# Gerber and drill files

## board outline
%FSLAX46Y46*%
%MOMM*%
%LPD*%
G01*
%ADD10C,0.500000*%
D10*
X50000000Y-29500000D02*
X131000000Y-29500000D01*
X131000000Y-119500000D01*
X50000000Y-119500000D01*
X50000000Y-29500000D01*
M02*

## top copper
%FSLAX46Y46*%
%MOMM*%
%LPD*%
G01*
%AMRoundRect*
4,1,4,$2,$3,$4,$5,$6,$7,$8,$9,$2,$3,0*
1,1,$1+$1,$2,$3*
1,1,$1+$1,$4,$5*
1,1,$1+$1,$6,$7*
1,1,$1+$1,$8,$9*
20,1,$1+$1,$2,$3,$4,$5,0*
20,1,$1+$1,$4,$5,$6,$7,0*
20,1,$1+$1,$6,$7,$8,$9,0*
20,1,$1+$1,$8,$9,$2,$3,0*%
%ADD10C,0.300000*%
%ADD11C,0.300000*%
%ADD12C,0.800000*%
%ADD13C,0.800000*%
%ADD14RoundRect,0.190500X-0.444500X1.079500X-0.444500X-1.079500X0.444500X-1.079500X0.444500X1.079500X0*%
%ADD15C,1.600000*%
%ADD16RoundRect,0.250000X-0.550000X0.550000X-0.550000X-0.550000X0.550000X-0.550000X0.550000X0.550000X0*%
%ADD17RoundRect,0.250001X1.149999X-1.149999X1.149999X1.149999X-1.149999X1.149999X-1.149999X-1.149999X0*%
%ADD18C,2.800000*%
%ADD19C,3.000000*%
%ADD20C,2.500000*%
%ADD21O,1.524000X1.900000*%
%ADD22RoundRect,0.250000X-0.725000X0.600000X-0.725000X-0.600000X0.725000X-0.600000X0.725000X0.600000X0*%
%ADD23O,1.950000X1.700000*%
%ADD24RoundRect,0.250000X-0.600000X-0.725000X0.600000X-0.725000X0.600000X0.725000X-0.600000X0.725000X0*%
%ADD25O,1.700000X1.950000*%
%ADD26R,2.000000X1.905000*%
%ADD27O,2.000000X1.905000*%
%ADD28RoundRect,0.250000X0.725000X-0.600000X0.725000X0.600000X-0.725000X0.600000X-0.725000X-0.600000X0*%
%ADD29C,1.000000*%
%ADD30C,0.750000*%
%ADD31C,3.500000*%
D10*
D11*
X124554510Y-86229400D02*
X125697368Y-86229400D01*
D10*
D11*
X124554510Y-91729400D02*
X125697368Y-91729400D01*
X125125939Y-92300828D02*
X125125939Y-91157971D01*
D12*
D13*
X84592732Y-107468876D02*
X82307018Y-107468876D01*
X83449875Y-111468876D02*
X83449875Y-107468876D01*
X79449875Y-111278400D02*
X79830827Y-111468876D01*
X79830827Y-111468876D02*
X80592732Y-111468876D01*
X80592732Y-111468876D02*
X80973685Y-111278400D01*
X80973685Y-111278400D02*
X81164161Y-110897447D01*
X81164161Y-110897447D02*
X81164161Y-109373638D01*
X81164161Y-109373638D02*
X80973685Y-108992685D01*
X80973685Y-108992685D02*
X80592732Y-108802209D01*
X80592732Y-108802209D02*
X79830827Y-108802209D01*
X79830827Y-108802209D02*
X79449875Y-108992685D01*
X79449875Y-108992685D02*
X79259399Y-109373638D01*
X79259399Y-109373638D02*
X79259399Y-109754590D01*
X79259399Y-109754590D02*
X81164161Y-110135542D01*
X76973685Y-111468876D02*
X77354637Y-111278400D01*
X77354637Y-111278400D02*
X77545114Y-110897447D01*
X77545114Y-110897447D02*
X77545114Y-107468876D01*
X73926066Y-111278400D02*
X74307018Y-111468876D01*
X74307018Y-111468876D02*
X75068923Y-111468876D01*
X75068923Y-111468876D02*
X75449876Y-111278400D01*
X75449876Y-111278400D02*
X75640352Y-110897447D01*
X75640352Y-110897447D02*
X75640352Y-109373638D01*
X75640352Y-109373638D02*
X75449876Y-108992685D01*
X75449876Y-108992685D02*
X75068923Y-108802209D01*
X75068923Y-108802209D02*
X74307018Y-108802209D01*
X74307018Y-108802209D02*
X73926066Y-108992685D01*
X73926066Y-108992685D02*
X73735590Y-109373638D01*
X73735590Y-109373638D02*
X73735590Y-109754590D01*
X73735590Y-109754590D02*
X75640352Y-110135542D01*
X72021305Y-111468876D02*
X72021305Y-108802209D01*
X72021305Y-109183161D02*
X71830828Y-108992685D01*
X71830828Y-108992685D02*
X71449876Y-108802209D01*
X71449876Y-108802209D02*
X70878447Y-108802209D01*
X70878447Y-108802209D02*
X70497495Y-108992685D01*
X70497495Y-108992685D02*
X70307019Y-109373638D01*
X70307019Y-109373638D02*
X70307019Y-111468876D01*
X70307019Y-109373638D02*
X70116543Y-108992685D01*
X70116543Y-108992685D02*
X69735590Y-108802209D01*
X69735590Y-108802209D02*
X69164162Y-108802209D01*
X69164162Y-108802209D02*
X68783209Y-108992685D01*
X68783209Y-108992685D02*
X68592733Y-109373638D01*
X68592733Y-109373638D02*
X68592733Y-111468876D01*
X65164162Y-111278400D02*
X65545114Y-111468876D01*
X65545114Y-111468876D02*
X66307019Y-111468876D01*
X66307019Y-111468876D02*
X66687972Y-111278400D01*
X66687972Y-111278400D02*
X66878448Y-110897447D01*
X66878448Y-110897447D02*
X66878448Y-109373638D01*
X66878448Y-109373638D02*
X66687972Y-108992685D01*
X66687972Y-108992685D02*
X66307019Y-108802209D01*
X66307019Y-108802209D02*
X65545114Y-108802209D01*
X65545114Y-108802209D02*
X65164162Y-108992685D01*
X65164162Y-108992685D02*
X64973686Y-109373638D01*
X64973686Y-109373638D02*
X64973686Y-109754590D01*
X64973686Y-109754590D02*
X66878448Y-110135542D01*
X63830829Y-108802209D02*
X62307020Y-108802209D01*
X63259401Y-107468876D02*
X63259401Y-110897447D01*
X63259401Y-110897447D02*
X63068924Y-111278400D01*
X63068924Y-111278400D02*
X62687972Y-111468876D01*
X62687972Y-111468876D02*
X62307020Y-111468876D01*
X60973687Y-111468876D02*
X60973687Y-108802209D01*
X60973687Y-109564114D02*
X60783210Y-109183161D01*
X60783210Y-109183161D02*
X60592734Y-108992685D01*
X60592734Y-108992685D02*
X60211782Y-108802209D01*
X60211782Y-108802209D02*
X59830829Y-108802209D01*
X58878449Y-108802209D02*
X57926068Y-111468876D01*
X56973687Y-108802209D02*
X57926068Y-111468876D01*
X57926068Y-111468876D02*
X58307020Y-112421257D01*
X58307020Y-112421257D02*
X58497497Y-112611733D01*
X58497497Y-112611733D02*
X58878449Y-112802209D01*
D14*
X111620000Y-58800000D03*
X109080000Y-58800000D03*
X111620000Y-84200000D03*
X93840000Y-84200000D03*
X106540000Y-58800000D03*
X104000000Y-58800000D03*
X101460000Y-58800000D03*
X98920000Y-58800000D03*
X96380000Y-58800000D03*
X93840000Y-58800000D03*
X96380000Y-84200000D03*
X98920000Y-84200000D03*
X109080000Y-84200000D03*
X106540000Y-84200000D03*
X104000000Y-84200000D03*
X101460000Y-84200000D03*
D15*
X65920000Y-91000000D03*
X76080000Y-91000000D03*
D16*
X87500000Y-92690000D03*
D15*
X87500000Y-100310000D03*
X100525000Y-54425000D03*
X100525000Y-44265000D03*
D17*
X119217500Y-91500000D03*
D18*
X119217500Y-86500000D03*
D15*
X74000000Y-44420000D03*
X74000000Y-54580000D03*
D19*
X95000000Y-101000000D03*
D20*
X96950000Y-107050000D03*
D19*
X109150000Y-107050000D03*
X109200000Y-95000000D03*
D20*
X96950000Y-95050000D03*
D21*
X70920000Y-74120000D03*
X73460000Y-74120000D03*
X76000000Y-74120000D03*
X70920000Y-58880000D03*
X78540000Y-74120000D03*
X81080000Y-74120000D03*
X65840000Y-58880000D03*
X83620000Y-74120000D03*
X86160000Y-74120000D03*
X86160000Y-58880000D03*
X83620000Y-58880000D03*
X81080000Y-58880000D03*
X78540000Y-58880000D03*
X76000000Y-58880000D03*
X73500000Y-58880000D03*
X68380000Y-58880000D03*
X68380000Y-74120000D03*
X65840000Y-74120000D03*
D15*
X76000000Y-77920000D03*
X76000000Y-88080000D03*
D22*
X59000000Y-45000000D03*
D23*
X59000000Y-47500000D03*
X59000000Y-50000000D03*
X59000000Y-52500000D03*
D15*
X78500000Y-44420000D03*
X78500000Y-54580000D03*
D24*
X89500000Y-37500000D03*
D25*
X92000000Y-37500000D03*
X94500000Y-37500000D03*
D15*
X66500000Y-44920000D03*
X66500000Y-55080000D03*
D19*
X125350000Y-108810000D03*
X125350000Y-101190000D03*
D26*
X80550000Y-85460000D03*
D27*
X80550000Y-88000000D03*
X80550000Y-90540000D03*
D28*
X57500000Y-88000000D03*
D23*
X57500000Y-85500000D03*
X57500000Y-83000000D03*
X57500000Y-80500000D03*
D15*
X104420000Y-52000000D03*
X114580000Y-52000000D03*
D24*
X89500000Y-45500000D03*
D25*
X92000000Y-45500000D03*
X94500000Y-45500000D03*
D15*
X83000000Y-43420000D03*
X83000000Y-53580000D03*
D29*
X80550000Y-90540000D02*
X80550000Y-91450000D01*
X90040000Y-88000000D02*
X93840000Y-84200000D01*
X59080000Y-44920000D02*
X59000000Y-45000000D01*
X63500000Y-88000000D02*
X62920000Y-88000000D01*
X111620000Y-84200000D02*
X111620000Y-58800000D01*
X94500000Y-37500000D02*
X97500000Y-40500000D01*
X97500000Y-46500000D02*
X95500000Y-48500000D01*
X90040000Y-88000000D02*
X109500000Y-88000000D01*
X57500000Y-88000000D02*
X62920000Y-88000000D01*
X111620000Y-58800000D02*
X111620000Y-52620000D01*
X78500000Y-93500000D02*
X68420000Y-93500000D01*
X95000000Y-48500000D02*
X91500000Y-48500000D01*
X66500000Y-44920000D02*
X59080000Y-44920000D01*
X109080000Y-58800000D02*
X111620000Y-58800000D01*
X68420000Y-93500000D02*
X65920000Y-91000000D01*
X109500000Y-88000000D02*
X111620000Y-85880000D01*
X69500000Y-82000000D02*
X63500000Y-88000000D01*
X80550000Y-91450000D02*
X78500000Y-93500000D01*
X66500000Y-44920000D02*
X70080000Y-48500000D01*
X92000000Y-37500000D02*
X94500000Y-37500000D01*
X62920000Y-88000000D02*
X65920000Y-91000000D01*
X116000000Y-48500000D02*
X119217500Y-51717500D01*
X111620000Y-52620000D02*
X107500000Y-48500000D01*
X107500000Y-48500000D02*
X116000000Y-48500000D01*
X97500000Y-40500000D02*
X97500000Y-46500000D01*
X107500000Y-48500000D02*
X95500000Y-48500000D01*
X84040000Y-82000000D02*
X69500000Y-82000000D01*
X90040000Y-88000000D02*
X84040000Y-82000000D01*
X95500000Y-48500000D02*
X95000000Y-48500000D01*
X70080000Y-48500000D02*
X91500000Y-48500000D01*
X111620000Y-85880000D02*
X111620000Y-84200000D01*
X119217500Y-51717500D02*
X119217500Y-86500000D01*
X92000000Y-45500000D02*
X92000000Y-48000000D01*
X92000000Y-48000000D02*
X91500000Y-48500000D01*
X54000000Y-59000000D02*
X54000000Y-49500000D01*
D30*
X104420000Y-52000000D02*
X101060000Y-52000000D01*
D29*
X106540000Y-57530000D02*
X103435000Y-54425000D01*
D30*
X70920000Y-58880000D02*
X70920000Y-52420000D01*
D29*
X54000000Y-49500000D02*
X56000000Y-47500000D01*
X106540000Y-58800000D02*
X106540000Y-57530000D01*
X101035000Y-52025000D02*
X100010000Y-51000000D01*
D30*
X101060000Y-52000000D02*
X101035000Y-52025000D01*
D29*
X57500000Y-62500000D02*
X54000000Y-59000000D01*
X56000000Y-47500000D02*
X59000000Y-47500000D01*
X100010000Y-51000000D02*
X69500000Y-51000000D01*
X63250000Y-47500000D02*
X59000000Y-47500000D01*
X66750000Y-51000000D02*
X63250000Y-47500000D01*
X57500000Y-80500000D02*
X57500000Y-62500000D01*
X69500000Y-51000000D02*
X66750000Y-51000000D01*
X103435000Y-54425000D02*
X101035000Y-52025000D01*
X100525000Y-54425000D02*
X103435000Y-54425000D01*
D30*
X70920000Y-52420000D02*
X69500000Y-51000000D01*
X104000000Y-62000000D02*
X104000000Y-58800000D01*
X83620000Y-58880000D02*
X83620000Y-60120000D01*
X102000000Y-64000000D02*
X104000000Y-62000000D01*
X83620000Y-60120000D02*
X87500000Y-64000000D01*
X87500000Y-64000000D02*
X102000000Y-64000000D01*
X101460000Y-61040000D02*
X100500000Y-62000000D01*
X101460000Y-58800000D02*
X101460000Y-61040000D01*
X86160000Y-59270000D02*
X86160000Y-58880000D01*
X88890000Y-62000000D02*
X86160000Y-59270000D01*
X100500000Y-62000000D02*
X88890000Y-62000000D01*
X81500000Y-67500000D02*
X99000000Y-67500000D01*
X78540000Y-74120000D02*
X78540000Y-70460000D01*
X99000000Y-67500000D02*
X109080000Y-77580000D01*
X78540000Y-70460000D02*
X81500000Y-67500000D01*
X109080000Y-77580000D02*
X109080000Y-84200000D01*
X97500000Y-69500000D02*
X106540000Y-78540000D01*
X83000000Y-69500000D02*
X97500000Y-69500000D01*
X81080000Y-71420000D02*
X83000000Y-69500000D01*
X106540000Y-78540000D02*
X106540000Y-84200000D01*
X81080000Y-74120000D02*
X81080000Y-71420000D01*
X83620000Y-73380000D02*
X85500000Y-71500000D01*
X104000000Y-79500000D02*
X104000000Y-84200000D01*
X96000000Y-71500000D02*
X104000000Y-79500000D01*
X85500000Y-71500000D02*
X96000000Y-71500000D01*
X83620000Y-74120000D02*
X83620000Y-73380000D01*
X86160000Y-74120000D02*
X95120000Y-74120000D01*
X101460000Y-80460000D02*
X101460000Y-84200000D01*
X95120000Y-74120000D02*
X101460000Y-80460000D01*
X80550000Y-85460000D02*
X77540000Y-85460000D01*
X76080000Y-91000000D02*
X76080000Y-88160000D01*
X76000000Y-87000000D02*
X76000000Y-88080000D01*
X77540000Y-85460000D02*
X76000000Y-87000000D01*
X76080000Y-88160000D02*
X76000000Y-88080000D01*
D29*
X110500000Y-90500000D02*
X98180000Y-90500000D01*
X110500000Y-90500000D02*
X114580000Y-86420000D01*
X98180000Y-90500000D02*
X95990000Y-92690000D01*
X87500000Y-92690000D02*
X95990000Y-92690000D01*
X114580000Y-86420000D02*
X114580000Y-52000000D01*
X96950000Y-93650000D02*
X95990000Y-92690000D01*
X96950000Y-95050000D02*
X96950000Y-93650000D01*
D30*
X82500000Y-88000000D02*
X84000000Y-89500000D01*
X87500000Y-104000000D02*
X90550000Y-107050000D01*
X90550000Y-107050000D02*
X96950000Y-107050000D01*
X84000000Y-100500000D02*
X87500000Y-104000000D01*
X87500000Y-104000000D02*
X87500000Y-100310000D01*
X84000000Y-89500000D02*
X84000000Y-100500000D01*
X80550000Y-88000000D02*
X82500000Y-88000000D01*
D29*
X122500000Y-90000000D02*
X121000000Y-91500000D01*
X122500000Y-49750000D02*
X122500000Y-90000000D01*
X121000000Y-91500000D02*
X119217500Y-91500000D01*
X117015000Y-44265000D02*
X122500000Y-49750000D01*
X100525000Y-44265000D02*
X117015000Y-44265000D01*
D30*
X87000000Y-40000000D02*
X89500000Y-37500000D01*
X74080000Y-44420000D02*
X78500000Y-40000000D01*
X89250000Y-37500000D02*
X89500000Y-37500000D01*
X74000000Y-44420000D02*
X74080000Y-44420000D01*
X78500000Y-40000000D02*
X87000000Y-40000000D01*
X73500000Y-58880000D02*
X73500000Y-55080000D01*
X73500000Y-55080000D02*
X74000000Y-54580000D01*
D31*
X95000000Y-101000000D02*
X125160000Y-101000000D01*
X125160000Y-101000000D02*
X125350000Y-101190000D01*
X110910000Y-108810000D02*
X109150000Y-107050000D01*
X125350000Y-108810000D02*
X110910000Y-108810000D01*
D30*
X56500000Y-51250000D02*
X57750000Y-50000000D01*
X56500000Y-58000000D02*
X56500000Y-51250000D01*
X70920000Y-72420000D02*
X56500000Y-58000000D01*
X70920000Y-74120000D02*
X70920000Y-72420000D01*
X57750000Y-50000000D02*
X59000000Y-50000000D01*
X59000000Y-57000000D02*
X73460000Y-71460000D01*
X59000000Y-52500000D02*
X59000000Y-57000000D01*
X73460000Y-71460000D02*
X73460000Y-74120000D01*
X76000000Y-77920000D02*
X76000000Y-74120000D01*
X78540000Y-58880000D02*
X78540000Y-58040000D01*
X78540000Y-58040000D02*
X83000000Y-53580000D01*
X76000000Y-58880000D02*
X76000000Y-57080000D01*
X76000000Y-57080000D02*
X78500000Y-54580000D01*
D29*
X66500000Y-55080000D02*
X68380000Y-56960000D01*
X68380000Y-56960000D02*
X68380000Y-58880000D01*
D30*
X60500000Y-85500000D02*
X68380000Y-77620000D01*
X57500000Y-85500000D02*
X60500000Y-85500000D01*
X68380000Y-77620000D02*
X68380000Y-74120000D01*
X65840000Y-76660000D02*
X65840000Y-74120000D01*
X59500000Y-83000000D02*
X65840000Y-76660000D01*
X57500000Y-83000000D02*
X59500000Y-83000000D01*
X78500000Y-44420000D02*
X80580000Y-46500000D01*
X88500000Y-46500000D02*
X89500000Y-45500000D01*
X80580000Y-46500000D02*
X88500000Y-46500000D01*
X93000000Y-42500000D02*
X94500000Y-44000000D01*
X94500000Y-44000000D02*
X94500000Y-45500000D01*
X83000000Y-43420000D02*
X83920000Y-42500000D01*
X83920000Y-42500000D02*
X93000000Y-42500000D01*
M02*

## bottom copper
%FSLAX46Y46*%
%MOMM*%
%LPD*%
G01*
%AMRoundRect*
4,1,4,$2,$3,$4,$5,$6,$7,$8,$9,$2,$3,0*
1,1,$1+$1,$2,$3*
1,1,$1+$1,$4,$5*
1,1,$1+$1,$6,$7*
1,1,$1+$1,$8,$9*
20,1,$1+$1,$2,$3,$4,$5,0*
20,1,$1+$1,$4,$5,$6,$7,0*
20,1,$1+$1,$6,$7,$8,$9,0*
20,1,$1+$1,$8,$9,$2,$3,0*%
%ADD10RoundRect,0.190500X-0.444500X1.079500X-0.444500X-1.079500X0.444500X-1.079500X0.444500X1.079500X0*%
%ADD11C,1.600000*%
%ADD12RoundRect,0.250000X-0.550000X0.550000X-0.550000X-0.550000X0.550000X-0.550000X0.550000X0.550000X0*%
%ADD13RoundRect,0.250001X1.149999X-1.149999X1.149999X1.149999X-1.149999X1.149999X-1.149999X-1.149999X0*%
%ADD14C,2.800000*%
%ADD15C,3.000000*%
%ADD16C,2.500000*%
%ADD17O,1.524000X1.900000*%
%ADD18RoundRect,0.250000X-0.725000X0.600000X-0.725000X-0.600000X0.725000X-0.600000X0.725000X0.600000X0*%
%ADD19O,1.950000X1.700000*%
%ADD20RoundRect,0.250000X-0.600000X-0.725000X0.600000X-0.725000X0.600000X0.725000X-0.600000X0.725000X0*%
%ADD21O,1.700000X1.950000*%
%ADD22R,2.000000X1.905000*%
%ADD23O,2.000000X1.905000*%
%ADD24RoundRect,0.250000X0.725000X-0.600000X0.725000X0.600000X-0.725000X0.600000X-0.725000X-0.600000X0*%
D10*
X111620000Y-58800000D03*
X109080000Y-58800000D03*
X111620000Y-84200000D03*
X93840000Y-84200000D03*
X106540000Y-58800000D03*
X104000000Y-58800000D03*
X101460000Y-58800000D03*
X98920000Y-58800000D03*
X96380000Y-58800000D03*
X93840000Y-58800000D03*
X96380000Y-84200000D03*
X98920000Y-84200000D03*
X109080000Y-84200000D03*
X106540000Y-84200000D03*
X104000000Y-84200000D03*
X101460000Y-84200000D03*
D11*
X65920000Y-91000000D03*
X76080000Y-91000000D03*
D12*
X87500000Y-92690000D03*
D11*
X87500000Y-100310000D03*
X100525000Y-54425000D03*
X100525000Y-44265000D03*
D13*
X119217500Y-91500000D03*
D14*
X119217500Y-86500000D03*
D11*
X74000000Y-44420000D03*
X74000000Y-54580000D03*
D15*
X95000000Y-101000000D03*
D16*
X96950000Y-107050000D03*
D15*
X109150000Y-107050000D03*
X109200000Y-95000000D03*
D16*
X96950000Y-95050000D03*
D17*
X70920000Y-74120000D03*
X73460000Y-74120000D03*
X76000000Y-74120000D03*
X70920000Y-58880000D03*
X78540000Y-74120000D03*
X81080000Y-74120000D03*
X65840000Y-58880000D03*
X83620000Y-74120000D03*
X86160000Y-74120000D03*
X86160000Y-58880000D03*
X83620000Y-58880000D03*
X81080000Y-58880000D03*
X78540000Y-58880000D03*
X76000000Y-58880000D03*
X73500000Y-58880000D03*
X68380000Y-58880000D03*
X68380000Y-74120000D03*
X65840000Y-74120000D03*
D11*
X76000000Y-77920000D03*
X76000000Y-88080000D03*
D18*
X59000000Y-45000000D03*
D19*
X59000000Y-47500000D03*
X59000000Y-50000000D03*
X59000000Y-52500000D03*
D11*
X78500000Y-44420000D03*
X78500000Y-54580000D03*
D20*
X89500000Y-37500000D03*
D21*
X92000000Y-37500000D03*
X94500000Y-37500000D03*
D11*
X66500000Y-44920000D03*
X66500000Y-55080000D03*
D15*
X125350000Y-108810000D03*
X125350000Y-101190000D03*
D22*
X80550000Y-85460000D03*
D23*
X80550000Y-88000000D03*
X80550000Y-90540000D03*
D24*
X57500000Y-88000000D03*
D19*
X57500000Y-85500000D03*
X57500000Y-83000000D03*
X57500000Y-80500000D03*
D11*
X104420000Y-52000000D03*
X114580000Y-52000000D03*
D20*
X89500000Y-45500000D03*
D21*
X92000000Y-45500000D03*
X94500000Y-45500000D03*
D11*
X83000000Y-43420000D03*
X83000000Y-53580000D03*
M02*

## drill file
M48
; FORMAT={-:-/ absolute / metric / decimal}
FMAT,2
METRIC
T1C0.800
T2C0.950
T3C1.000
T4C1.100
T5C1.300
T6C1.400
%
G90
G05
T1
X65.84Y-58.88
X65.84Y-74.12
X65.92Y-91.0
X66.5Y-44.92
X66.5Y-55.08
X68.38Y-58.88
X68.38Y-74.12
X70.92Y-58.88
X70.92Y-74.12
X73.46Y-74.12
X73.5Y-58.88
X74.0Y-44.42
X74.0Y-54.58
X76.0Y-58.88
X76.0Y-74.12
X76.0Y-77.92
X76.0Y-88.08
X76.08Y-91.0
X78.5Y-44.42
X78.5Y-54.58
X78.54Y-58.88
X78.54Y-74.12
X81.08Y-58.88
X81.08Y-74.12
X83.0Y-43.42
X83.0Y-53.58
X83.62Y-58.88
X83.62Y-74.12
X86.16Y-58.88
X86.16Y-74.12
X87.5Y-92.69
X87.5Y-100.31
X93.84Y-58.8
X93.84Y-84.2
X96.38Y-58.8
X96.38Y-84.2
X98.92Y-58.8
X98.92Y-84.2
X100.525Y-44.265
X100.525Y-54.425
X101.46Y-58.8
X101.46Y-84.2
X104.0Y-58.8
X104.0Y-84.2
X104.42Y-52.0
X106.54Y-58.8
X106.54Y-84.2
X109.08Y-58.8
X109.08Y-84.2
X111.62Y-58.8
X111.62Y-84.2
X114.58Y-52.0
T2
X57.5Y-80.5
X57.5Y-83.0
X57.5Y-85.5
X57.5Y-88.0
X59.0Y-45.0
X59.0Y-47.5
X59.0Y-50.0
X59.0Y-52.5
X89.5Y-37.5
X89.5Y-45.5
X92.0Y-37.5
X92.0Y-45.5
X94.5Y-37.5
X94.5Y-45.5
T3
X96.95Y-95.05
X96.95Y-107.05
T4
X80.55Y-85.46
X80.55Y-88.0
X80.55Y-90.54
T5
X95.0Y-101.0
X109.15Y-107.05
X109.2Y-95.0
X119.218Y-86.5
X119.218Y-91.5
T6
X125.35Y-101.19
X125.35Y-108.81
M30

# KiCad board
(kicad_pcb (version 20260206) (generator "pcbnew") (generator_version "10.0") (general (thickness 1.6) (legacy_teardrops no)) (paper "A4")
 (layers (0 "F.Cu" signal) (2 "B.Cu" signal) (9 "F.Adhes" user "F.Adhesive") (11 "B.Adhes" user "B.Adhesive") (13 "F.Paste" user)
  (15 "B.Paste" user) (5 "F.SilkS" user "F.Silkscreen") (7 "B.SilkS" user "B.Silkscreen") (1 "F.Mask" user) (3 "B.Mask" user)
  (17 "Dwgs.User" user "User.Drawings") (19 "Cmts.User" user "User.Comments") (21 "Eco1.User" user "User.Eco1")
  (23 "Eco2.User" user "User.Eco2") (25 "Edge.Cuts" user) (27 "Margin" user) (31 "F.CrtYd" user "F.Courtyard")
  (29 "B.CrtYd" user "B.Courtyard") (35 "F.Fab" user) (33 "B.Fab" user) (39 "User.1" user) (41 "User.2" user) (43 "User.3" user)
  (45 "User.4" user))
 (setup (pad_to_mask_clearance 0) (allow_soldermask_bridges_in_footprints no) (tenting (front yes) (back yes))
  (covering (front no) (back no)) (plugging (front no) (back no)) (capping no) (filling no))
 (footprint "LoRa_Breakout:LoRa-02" (layer "F.Cu") (at 101.46 71.5 -90)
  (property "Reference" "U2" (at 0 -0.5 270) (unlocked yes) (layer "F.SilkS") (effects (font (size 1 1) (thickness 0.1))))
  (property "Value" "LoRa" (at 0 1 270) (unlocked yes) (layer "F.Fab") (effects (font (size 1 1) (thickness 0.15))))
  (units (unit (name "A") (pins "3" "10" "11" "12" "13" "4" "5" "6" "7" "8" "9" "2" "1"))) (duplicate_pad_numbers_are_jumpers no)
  (pad "1" thru_hole roundrect (at -12.7 -10.16 270) (size 2.54 1.27) (drill 0.8) (layers "*.Cu" "*.Mask") (remove_unused_layers no)
   (roundrect_rratio 0.15) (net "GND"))
  (pad "1" thru_hole roundrect (at -12.7 -7.62 270) (size 2.54 1.27) (drill 0.8) (layers "*.Cu" "*.Mask") (remove_unused_layers no)
   (roundrect_rratio 0.15) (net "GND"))
  (pad "1" thru_hole roundrect (at 12.7 -10.16 270) (size 2.54 1.27) (drill 0.8) (layers "*.Cu" "*.Mask") (remove_unused_layers no)
   (roundrect_rratio 0.15) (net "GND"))
  (pad "1" thru_hole roundrect (at 12.7 7.62 270) (size 2.54 1.27) (drill 0.8) (layers "*.Cu" "*.Mask") (remove_unused_layers no)
   (roundrect_rratio 0.15) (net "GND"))
  (pad "2" thru_hole roundrect (at -12.7 -5.08 270) (size 2.54 1.27) (drill 0.8) (layers "*.Cu" "*.Mask") (remove_unused_layers no)
   (roundrect_rratio 0.15) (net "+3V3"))
  (pad "3" thru_hole roundrect (at -12.7 -2.54 270) (size 2.54 1.27) (drill 0.8) (layers "*.Cu" "*.Mask") (remove_unused_layers no)
   (roundrect_rratio 0.15) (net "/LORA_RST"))
  (pad "4" thru_hole roundrect (at -12.7 0 270) (size 2.54 1.27) (drill 0.8) (layers "*.Cu" "*.Mask") (remove_unused_layers no)
   (roundrect_rratio 0.15) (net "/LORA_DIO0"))
  (pad "5" thru_hole roundrect (at -12.7 2.54 270) (size 2.54 1.27) (drill 0.8) (layers "*.Cu" "*.Mask") (remove_unused_layers no)
   (roundrect_rratio 0.15) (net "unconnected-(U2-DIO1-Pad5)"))
  (pad "6" thru_hole roundrect (at -12.7 5.08 270) (size 2.54 1.27) (drill 0.8) (layers "*.Cu" "*.Mask") (remove_unused_layers no)
   (roundrect_rratio 0.15) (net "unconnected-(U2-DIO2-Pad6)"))
  (pad "7" thru_hole roundrect (at -12.7 7.62 270) (size 2.54 1.27) (drill 0.8) (layers "*.Cu" "*.Mask") (remove_unused_layers no)
   (roundrect_rratio 0.15) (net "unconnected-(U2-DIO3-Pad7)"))
  (pad "8" thru_hole roundrect (at 12.7 5.08 270) (size 2.54 1.27) (drill 0.8) (layers "*.Cu" "*.Mask") (remove_unused_layers no)
   (roundrect_rratio 0.15) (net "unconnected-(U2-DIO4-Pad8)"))
  (pad "9" thru_hole roundrect (at 12.7 2.54 270) (size 2.54 1.27) (drill 0.8) (layers "*.Cu" "*.Mask") (remove_unused_layers no)
   (roundrect_rratio 0.15) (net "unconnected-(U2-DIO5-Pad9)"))
  (pad "10" thru_hole roundrect (at 12.7 -7.62 270) (size 2.54 1.27) (drill 0.8) (layers "*.Cu" "*.Mask") (remove_unused_layers no)
   (roundrect_rratio 0.15) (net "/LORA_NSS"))
  (pad "11" thru_hole roundrect (at 12.7 -5.08 270) (size 2.54 1.27) (drill 0.8) (layers "*.Cu" "*.Mask") (remove_unused_layers no)
   (roundrect_rratio 0.15) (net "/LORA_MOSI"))
  (pad "12" thru_hole roundrect (at 12.7 -2.54 270) (size 2.54 1.27) (drill 0.8) (layers "*.Cu" "*.Mask") (remove_unused_layers no)
   (roundrect_rratio 0.15) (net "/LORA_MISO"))
  (pad "13" thru_hole roundrect (at 12.7 0 270) (size 2.54 1.27) (drill 0.8) (layers "*.Cu" "*.Mask") (remove_unused_layers no)
   (roundrect_rratio 0.15) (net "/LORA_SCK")))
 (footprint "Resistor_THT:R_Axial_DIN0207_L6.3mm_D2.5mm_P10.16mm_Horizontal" (layer "F.Cu") (at 65.92 91)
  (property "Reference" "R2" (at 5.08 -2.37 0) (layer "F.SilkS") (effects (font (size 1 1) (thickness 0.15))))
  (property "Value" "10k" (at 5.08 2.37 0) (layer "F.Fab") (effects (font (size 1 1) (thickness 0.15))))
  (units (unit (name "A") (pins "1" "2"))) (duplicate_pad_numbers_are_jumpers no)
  (pad "1" thru_hole circle (at 0 0) (size 1.6 1.6) (drill 0.8) (layers "*.Cu" "*.Mask") (remove_unused_layers no) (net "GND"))
  (pad "2" thru_hole circle (at 10.16 0) (size 1.6 1.6) (drill 0.8) (layers "*.Cu" "*.Mask") (remove_unused_layers no) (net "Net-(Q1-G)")))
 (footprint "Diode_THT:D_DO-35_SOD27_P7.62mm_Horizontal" (layer "F.Cu") (at 87.5 92.69 -90)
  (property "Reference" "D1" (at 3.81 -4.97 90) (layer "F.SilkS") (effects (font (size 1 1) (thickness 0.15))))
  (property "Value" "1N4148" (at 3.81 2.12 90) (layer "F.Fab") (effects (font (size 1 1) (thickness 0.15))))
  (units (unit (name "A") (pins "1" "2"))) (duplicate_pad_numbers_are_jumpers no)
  (pad "1" thru_hole roundrect (at 0 0 270) (size 1.6 1.6) (drill 0.8) (layers "*.Cu" "*.Mask") (remove_unused_layers no)
   (roundrect_rratio 0.15625) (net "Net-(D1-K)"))
  (pad "2" thru_hole circle (at 7.62 0 270) (size 1.6 1.6) (drill 0.8) (layers "*.Cu" "*.Mask") (remove_unused_layers no) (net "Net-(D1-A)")))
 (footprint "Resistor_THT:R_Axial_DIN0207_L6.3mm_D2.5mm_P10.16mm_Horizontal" (layer "F.Cu") (at 100.525 54.425 90)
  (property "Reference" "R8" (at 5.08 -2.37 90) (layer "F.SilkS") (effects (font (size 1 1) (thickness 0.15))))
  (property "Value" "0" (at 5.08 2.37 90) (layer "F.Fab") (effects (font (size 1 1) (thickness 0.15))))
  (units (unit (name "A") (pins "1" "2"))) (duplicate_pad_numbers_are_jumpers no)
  (pad "1" thru_hole circle (at 0 0 90) (size 1.6 1.6) (drill 0.8) (layers "*.Cu" "*.Mask") (remove_unused_layers no) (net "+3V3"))
  (pad "2" thru_hole circle (at 10.16 0 90) (size 1.6 1.6) (drill 0.8) (layers "*.Cu" "*.Mask") (remove_unused_layers no)
   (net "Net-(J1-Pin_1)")))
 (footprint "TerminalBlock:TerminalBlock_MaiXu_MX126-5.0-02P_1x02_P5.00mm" (layer "F.Cu") (at 119.2175 91.5 90)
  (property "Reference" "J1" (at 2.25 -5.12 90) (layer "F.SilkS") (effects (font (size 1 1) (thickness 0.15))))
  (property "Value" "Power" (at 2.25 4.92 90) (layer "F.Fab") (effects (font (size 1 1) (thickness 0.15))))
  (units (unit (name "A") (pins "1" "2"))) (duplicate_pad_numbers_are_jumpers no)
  (pad "1" thru_hole roundrect (at 0 0 90) (size 2.8 2.8) (drill 1.3) (layers "*.Cu" "*.Mask") (remove_unused_layers no)
   (roundrect_rratio 0.089286) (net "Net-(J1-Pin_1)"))
  (pad "2" thru_hole circle (at 5 0 90) (size 2.8 2.8) (drill 1.3) (layers "*.Cu" "*.Mask") (remove_unused_layers no) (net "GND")))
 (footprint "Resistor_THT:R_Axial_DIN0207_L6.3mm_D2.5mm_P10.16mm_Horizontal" (layer "F.Cu") (at 74 44.42 -90)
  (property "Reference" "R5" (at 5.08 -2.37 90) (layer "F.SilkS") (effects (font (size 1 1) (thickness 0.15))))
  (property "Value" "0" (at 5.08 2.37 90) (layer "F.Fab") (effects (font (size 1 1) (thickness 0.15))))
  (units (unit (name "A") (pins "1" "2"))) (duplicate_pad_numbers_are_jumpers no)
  (pad "1" thru_hole circle (at 0 0 270) (size 1.6 1.6) (drill 0.8) (layers "*.Cu" "*.Mask") (remove_unused_layers no)
   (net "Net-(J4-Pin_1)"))
  (pad "2" thru_hole circle (at 10.16 0 270) (size 1.6 1.6) (drill 0.8) (layers "*.Cu" "*.Mask") (remove_unused_layers no)
   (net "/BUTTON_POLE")))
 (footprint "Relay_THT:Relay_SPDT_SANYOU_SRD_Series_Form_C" (layer "F.Cu") (at 95 101)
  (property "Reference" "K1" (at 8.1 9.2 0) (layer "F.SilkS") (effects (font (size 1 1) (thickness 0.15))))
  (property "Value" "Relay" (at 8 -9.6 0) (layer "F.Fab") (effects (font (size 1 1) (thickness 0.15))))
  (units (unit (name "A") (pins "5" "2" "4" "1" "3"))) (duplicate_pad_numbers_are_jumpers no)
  (pad "1" thru_hole circle (at 0 0 90) (size 3 3) (drill 1.3) (layers "*.Cu" "*.Mask") (remove_unused_layers no) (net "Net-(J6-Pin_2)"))
  (pad "2" thru_hole circle (at 1.95 6.05 90) (size 2.5 2.5) (drill 1) (layers "*.Cu" "*.Mask") (remove_unused_layers no) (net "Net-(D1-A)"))
  (pad "3" thru_hole circle (at 14.15 6.05 90) (size 3 3) (drill 1.3) (layers "*.Cu" "*.Mask") (remove_unused_layers no)
   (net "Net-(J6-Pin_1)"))
  (pad "4" thru_hole circle (at 14.2 -6 90) (size 3 3) (drill 1.3) (layers "*.Cu" "*.Mask") (remove_unused_layers no)
   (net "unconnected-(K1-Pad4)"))
  (pad "5" thru_hole circle (at 1.95 -5.95 90) (size 2.5 2.5) (drill 1) (layers "*.Cu" "*.Mask") (remove_unused_layers no)
   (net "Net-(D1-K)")))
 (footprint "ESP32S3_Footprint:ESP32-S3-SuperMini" (layer "F.Cu") (at 76 66.5 90)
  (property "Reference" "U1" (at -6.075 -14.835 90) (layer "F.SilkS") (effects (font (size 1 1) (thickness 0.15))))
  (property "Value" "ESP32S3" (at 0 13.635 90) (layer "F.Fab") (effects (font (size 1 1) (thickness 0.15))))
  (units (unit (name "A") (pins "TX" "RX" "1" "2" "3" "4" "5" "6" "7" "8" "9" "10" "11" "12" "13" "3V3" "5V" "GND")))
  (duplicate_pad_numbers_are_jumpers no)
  (pad "1" thru_hole oval (at -7.62 -5.08) (size 1.524 1.9) (drill 0.8) (layers "*.Cu" "*.Mask") (remove_unused_layers no) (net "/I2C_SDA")
   (solder_mask_margin 0.102))
  (pad "2" thru_hole oval (at -7.62 -2.54) (size 1.524 1.9) (drill 0.8) (layers "*.Cu" "*.Mask") (remove_unused_layers no) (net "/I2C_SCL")
   (solder_mask_margin 0.102) (thermal_bridge_angle 45))
  (pad "3" thru_hole oval (at -7.62 0) (size 1.524 1.9) (drill 0.8) (layers "*.Cu" "*.Mask") (remove_unused_layers no) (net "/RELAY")
   (solder_mask_margin 0.102) (thermal_bridge_angle 45))
  (pad "3V3" thru_hole oval (at 7.62 -5.08) (size 1.524 1.9) (drill 0.8) (layers "*.Cu" "*.Mask") (remove_unused_layers no) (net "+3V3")
   (solder_mask_margin 0.102) (thermal_bridge_angle 45))
  (pad "4" thru_hole oval (at -7.62 2.54) (size 1.524 1.9) (drill 0.8) (layers "*.Cu" "*.Mask") (remove_unused_layers no) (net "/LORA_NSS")
   (solder_mask_margin 0.102) (thermal_bridge_angle 45))
  (pad "5" thru_hole oval (at -7.62 5.08) (size 1.524 1.9) (drill 0.8) (layers "*.Cu" "*.Mask") (remove_unused_layers no) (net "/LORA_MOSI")
   (solder_mask_margin 0.102) (thermal_bridge_angle 45))
  (pad "5V" thru_hole oval (at 7.62 -10.16) (size 1.524 1.9) (drill 0.8) (layers "*.Cu" "*.Mask") (remove_unused_layers no)
   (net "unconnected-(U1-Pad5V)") (solder_mask_margin 0.102))
  (pad "6" thru_hole oval (at -7.62 7.62) (size 1.524 1.9) (drill 0.8) (layers "*.Cu" "*.Mask") (remove_unused_layers no) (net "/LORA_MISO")
   (solder_mask_margin 0.102) (thermal_bridge_angle 45))
  (pad "7" thru_hole oval (at -7.62 10.16) (size 1.524 1.9) (drill 0.8) (layers "*.Cu" "*.Mask") (remove_unused_layers no) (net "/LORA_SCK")
   (solder_mask_margin 0.102) (thermal_bridge_angle 45))
  (pad "8" thru_hole oval (at 7.62 10.16) (size 1.524 1.9) (drill 0.8) (layers "*.Cu" "*.Mask") (remove_unused_layers no) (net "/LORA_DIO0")
   (solder_mask_margin 0.102) (thermal_bridge_angle 45))
  (pad "9" thru_hole oval (at 7.62 7.62) (size 1.524 1.9) (drill 0.8) (layers "*.Cu" "*.Mask") (remove_unused_layers no) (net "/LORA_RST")
   (solder_mask_margin 0.102) (thermal_bridge_angle 45))
  (pad "10" thru_hole oval (at 7.62 5.08) (size 1.524 1.9) (drill 0.8) (layers "*.Cu" "*.Mask") (remove_unused_layers no)
   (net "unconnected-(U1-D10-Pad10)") (solder_mask_margin 0.102) (thermal_bridge_angle 45))
  (pad "11" thru_hole oval (at 7.62 2.54) (size 1.524 1.9) (drill 0.8) (layers "*.Cu" "*.Mask") (remove_unused_layers no) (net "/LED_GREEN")
   (solder_mask_margin 0.102) (thermal_bridge_angle 45))
  (pad "12" thru_hole oval (at 7.62 0) (size 1.524 1.9) (drill 0.8) (layers "*.Cu" "*.Mask") (remove_unused_layers no) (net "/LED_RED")
   (solder_mask_margin 0.102) (thermal_bridge_angle 45))
  (pad "13" thru_hole oval (at 7.62 -2.5) (size 1.524 1.9) (drill 0.8) (layers "*.Cu" "*.Mask") (remove_unused_layers no)
   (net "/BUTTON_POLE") (solder_mask_margin 0.102) (thermal_bridge_angle 45))
  (pad "GND" thru_hole oval (at 7.62 -7.62) (size 1.524 1.9) (drill 0.8) (layers "*.Cu" "*.Mask") (remove_unused_layers no)
   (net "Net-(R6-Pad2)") (solder_mask_margin 0.102) (thermal_bridge_angle 45))
  (pad "RX" thru_hole oval (at -7.62 -7.62) (size 1.524 1.9) (drill 0.8) (layers "*.Cu" "*.Mask") (remove_unused_layers no) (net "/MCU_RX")
   (solder_mask_margin 0.102))
  (pad "TX" thru_hole oval (at -7.62 -10.16) (size 1.524 1.9) (drill 0.8) (layers "*.Cu" "*.Mask") (remove_unused_layers no) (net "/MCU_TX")
   (solder_mask_margin 0.102)))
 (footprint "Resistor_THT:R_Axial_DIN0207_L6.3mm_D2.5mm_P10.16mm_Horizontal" (layer "F.Cu") (at 76 77.92 -90)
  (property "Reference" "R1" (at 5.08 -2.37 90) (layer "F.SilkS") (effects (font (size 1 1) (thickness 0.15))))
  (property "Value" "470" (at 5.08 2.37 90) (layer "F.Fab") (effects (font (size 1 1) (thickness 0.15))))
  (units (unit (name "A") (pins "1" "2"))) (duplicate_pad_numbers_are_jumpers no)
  (pad "1" thru_hole circle (at 0 0 270) (size 1.6 1.6) (drill 0.8) (layers "*.Cu" "*.Mask") (remove_unused_layers no) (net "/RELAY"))
  (pad "2" thru_hole circle (at 10.16 0 270) (size 1.6 1.6) (drill 0.8) (layers "*.Cu" "*.Mask") (remove_unused_layers no)
   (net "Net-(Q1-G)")))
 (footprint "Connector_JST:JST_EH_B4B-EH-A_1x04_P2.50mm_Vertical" (layer "F.Cu") (at 59 45 -90)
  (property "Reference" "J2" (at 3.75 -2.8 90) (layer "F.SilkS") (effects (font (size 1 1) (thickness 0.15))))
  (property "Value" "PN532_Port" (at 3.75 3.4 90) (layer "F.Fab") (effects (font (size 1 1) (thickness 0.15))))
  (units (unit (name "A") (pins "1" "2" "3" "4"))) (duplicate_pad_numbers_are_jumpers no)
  (pad "1" thru_hole roundrect (at 0 0 270) (size 1.7 1.95) (drill 0.95) (layers "*.Cu" "*.Mask") (remove_unused_layers no)
   (roundrect_rratio 0.147059) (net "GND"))
  (pad "2" thru_hole oval (at 2.5 0 270) (size 1.7 1.95) (drill 0.95) (layers "*.Cu" "*.Mask") (remove_unused_layers no) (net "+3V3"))
  (pad "3" thru_hole oval (at 5 0 270) (size 1.7 1.95) (drill 0.95) (layers "*.Cu" "*.Mask") (remove_unused_layers no) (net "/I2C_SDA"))
  (pad "4" thru_hole oval (at 7.5 0 270) (size 1.7 1.95) (drill 0.95) (layers "*.Cu" "*.Mask") (remove_unused_layers no) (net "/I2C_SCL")))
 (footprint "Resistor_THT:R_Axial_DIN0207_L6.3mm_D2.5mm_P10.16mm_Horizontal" (layer "F.Cu") (at 78.5 44.42 -90)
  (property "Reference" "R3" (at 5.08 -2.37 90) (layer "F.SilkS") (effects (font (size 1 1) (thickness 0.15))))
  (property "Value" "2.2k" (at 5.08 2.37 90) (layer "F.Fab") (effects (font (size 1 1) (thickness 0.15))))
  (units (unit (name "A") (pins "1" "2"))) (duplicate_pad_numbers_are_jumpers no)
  (pad "1" thru_hole circle (at 0 0 270) (size 1.6 1.6) (drill 0.8) (layers "*.Cu" "*.Mask") (remove_unused_layers no)
   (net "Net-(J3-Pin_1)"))
  (pad "2" thru_hole circle (at 10.16 0 270) (size 1.6 1.6) (drill 0.8) (layers "*.Cu" "*.Mask") (remove_unused_layers no) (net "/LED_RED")))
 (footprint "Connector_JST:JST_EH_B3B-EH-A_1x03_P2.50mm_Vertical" (layer "F.Cu") (at 89.5 37.5)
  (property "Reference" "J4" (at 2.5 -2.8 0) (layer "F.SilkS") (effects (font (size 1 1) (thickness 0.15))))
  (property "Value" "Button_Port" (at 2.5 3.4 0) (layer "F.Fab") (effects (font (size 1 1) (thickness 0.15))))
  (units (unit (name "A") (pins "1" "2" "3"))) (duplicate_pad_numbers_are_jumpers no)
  (pad "1" thru_hole roundrect (at 0 0) (size 1.7 1.95) (drill 0.95) (layers "*.Cu" "*.Mask") (remove_unused_layers no)
   (roundrect_rratio 0.147059) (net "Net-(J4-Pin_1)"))
  (pad "2" thru_hole oval (at 2.5 0) (size 1.7 1.95) (drill 0.95) (layers "*.Cu" "*.Mask") (remove_unused_layers no) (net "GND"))
  (pad "3" thru_hole oval (at 5 0) (size 1.7 1.95) (drill 0.95) (layers "*.Cu" "*.Mask") (remove_unused_layers no) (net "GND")))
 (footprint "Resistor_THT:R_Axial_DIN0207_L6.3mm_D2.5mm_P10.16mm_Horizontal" (layer "F.Cu") (at 66.5 44.92 -90)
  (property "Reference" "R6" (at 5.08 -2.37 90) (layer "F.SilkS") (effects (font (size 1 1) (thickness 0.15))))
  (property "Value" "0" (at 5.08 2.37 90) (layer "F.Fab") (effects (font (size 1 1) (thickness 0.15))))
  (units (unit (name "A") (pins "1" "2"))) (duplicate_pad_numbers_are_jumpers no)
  (pad "1" thru_hole circle (at 0 0 270) (size 1.6 1.6) (drill 0.8) (layers "*.Cu" "*.Mask") (remove_unused_layers no) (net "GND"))
  (pad "2" thru_hole circle (at 10.16 0 270) (size 1.6 1.6) (drill 0.8) (layers "*.Cu" "*.Mask") (remove_unused_layers no)
   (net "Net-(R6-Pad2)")))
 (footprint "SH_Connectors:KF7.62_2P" (layer "F.Cu") (at 121.35 105 90)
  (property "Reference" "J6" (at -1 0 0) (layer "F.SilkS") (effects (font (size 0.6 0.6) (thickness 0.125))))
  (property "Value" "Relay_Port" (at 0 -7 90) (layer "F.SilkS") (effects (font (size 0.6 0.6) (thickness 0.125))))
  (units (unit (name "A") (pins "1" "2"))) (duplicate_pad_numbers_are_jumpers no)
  (pad "1" thru_hole circle (at -3.81 4 90) (size 3 3) (drill 1.4) (layers "*.Cu" "*.Mask" "F.SilkS") (remove_unused_layers no)
   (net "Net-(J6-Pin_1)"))
  (pad "2" thru_hole circle (at 3.81 4 90) (size 3 3) (drill 1.4) (layers "*.Cu" "*.Mask" "F.SilkS") (remove_unused_layers no)
   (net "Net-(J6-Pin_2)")))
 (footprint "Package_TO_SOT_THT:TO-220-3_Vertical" (layer "F.Cu") (at 80.55 85.46 -90)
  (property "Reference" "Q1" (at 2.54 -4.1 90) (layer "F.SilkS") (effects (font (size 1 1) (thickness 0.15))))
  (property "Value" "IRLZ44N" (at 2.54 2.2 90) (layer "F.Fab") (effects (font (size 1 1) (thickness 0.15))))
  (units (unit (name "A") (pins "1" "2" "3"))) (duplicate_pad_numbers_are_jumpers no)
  (pad "1" thru_hole rect (at 0 0 270) (size 1.905 2) (drill 1.1) (layers "*.Cu" "*.Mask") (remove_unused_layers no) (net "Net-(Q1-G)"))
  (pad "2" thru_hole oval (at 2.54 0 270) (size 1.905 2) (drill 1.1) (layers "*.Cu" "*.Mask") (remove_unused_layers no) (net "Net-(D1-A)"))
  (pad "3" thru_hole oval (at 5.08 0 270) (size 1.905 2) (drill 1.1) (layers "*.Cu" "*.Mask") (remove_unused_layers no) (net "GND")))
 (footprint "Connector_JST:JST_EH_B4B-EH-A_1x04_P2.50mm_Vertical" (layer "F.Cu") (at 57.5 88 90)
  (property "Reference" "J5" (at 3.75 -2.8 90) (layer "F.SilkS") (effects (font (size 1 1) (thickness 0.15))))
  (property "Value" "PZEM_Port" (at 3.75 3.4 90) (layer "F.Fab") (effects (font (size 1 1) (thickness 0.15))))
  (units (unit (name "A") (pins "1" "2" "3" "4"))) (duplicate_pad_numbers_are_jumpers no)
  (pad "1" thru_hole roundrect (at 0 0 90) (size 1.7 1.95) (drill 0.95) (layers "*.Cu" "*.Mask") (remove_unused_layers no)
   (roundrect_rratio 0.147059) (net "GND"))
  (pad "2" thru_hole oval (at 2.5 0 90) (size 1.7 1.95) (drill 0.95) (layers "*.Cu" "*.Mask") (remove_unused_layers no) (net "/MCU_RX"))
  (pad "3" thru_hole oval (at 5 0 90) (size 1.7 1.95) (drill 0.95) (layers "*.Cu" "*.Mask") (remove_unused_layers no) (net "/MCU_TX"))
  (pad "4" thru_hole oval (at 7.5 0 90) (size 1.7 1.95) (drill 0.95) (layers "*.Cu" "*.Mask") (remove_unused_layers no) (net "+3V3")))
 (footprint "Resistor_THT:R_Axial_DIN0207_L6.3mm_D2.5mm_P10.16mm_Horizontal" (layer "F.Cu") (at 104.42 52)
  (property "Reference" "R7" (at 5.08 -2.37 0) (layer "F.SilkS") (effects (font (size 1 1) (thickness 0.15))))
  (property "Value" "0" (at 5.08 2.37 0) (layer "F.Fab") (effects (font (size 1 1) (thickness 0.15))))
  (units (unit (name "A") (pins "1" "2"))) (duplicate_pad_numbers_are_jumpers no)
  (pad "1" thru_hole circle (at 0 0) (size 1.6 1.6) (drill 0.8) (layers "*.Cu" "*.Mask") (remove_unused_layers no) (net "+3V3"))
  (pad "2" thru_hole circle (at 10.16 0) (size 1.6 1.6) (drill 0.8) (layers "*.Cu" "*.Mask") (remove_unused_layers no) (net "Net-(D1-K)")))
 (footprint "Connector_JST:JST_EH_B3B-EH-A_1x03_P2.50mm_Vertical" (layer "F.Cu") (at 89.5 45.5)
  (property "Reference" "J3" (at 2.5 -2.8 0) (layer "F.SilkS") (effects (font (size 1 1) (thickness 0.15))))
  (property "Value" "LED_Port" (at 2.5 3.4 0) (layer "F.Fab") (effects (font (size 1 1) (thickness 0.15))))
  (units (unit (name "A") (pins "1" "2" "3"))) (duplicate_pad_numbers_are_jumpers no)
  (pad "1" thru_hole roundrect (at 0 0) (size 1.7 1.95) (drill 0.95) (layers "*.Cu" "*.Mask") (remove_unused_layers no)
   (roundrect_rratio 0.147059) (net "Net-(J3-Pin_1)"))
  (pad "2" thru_hole oval (at 2.5 0) (size 1.7 1.95) (drill 0.95) (layers "*.Cu" "*.Mask") (remove_unused_layers no) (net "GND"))
  (pad "3" thru_hole oval (at 5 0) (size 1.7 1.95) (drill 0.95) (layers "*.Cu" "*.Mask") (remove_unused_layers no) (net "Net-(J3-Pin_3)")))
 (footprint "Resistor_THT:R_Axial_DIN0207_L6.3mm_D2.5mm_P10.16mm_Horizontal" (layer "F.Cu") (at 83 43.42 -90)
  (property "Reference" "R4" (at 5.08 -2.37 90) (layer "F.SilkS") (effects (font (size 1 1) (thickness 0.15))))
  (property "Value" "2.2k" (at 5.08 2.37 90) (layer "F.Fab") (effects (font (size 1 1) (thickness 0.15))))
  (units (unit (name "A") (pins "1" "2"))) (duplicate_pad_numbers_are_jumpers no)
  (pad "1" thru_hole circle (at 0 0 270) (size 1.6 1.6) (drill 0.8) (layers "*.Cu" "*.Mask") (remove_unused_layers no)
   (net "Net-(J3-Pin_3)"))
  (pad "2" thru_hole circle (at 10.16 0 270) (size 1.6 1.6) (drill 0.8) (layers "*.Cu" "*.Mask") (remove_unused_layers no)
   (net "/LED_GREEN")))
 (gr_rect (start 50 29.5) (end 131 119.5) (stroke (width 0.5) (type solid)) (fill no) (layer "Edge.Cuts"))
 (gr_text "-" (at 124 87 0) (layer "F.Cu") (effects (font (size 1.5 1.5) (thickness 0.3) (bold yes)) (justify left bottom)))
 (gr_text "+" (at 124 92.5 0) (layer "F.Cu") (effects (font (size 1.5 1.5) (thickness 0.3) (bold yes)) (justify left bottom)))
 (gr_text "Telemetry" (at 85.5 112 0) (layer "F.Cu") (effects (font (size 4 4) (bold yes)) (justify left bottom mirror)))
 (segment (start 80.55 90.54) (end 80.55 91.45) (width 1) (layer "F.Cu") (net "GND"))
 (segment (start 90.04 88) (end 93.84 84.2) (width 1) (layer "F.Cu") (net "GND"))
 (segment (start 59.08 44.92) (end 59 45) (width 1) (layer "F.Cu") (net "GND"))
 (segment (start 63.5 88) (end 62.92 88) (width 1) (layer "F.Cu") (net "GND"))
 (segment (start 111.62 84.2) (end 111.62 58.8) (width 1) (layer "F.Cu") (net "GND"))
 (segment (start 94.5 37.5) (end 97.5 40.5) (width 1) (layer "F.Cu") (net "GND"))
 (segment (start 97.5 46.5) (end 95.5 48.5) (width 1) (layer "F.Cu") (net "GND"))
 (segment (start 90.04 88) (end 109.5 88) (width 1) (layer "F.Cu") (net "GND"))
 (segment (start 57.5 88) (end 62.92 88) (width 1) (layer "F.Cu") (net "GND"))
 (segment (start 111.62 58.8) (end 111.62 52.62) (width 1) (layer "F.Cu") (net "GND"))
 (segment (start 78.5 93.5) (end 68.42 93.5) (width 1) (layer "F.Cu") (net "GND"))
 (segment (start 95 48.5) (end 91.5 48.5) (width 1) (layer "F.Cu") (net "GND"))
 (segment (start 66.5 44.92) (end 59.08 44.92) (width 1) (layer "F.Cu") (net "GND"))
 (segment (start 109.08 58.8) (end 111.62 58.8) (width 1) (layer "F.Cu") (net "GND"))
 (segment (start 68.42 93.5) (end 65.92 91) (width 1) (layer "F.Cu") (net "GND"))
 (segment (start 109.5 88) (end 111.62 85.88) (width 1) (layer "F.Cu") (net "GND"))
 (segment (start 69.5 82) (end 63.5 88) (width 1) (layer "F.Cu") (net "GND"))
 (segment (start 80.55 91.45) (end 78.5 93.5) (width 1) (layer "F.Cu") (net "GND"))
 (segment (start 66.5 44.92) (end 70.08 48.5) (width 1) (layer "F.Cu") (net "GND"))
 (segment (start 92 37.5) (end 94.5 37.5) (width 1) (layer "F.Cu") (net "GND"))
 (segment (start 62.92 88) (end 65.92 91) (width 1) (layer "F.Cu") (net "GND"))
 (segment (start 116 48.5) (end 119.2175 51.7175) (width 1) (layer "F.Cu") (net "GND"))
 (segment (start 111.62 52.62) (end 107.5 48.5) (width 1) (layer "F.Cu") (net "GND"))
 (segment (start 107.5 48.5) (end 116 48.5) (width 1) (layer "F.Cu") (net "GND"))
 (segment (start 97.5 40.5) (end 97.5 46.5) (width 1) (layer "F.Cu") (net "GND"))
 (segment (start 107.5 48.5) (end 95.5 48.5) (width 1) (layer "F.Cu") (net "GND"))
 (segment (start 84.04 82) (end 69.5 82) (width 1) (layer "F.Cu") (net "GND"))
 (segment (start 90.04 88) (end 84.04 82) (width 1) (layer "F.Cu") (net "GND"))
 (segment (start 95.5 48.5) (end 95 48.5) (width 1) (layer "F.Cu") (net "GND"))
 (segment (start 70.08 48.5) (end 91.5 48.5) (width 1) (layer "F.Cu") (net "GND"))
 (segment (start 111.62 85.88) (end 111.62 84.2) (width 1) (layer "F.Cu") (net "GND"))
 (segment (start 119.2175 51.7175) (end 119.2175 86.5) (width 1) (layer "F.Cu") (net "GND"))
 (segment (start 92 45.5) (end 92 48) (width 1) (layer "F.Cu") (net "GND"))
 (segment (start 92 48) (end 91.5 48.5) (width 1) (layer "F.Cu") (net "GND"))
 (segment (start 54 59) (end 54 49.5) (width 1) (layer "F.Cu") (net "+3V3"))
 (segment (start 104.42 52) (end 101.06 52) (width 0.75) (layer "F.Cu") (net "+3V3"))
 (segment (start 106.54 57.53) (end 103.435 54.425) (width 1) (layer "F.Cu") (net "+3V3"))
 (segment (start 70.92 58.88) (end 70.92 52.42) (width 0.75) (layer "F.Cu") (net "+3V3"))
 (segment (start 54 49.5) (end 56 47.5) (width 1) (layer "F.Cu") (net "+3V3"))
 (segment (start 106.54 58.8) (end 106.54 57.53) (width 1) (layer "F.Cu") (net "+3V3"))
 (segment (start 101.035 52.025) (end 100.01 51) (width 1) (layer "F.Cu") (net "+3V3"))
 (segment (start 101.06 52) (end 101.035 52.025) (width 0.75) (layer "F.Cu") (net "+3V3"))
 (segment (start 57.5 62.5) (end 54 59) (width 1) (layer "F.Cu") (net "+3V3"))
 (segment (start 56 47.5) (end 59 47.5) (width 1) (layer "F.Cu") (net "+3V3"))
 (segment (start 100.01 51) (end 69.5 51) (width 1) (layer "F.Cu") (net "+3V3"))
 (segment (start 63.25 47.5) (end 59 47.5) (width 1) (layer "F.Cu") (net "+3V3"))
 (segment (start 66.75 51) (end 63.25 47.5) (width 1) (layer "F.Cu") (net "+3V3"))
 (segment (start 57.5 80.5) (end 57.5 62.5) (width 1) (layer "F.Cu") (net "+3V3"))
 (segment (start 69.5 51) (end 66.75 51) (width 1) (layer "F.Cu") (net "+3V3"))
 (segment (start 103.435 54.425) (end 101.035 52.025) (width 1) (layer "F.Cu") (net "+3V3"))
 (segment (start 100.525 54.425) (end 103.435 54.425) (width 1) (layer "F.Cu") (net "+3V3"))
 (segment (start 70.92 52.42) (end 69.5 51) (width 0.75) (layer "F.Cu") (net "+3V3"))
 (segment (start 104 62) (end 104 58.8) (width 0.75) (layer "F.Cu") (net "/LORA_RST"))
 (segment (start 83.62 58.88) (end 83.62 60.12) (width 0.75) (layer "F.Cu") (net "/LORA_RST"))
 (segment (start 102 64) (end 104 62) (width 0.75) (layer "F.Cu") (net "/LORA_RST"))
 (segment (start 83.62 60.12) (end 87.5 64) (width 0.75) (layer "F.Cu") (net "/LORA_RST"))
 (segment (start 87.5 64) (end 102 64) (width 0.75) (layer "F.Cu") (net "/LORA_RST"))
 (segment (start 101.46 61.04) (end 100.5 62) (width 0.75) (layer "F.Cu") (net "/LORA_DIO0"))
 (segment (start 101.46 58.8) (end 101.46 61.04) (width 0.75) (layer "F.Cu") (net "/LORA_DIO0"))
 (segment (start 86.16 59.27) (end 86.16 58.88) (width 0.75) (layer "F.Cu") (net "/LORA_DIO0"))
 (segment (start 88.89 62) (end 86.16 59.27) (width 0.75) (layer "F.Cu") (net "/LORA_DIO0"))
 (segment (start 100.5 62) (end 88.89 62) (width 0.75) (layer "F.Cu") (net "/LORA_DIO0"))
 (segment (start 81.5 67.5) (end 99 67.5) (width 0.75) (layer "F.Cu") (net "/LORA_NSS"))
 (segment (start 78.54 74.12) (end 78.54 70.46) (width 0.75) (layer "F.Cu") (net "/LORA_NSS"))
 (segment (start 99 67.5) (end 109.08 77.58) (width 0.75) (layer "F.Cu") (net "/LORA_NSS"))
 (segment (start 78.54 70.46) (end 81.5 67.5) (width 0.75) (layer "F.Cu") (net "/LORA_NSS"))
 (segment (start 109.08 77.58) (end 109.08 84.2) (width 0.75) (layer "F.Cu") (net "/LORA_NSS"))
 (segment (start 97.5 69.5) (end 106.54 78.54) (width 0.75) (layer "F.Cu") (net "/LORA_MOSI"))
 (segment (start 83 69.5) (end 97.5 69.5) (width 0.75) (layer "F.Cu") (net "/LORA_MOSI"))
 (segment (start 81.08 71.42) (end 83 69.5) (width 0.75) (layer "F.Cu") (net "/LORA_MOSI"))
 (segment (start 106.54 78.54) (end 106.54 84.2) (width 0.75) (layer "F.Cu") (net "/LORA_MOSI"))
 (segment (start 81.08 74.12) (end 81.08 71.42) (width 0.75) (layer "F.Cu") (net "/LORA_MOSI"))
 (segment (start 83.62 73.38) (end 85.5 71.5) (width 0.75) (layer "F.Cu") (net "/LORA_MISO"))
 (segment (start 104 79.5) (end 104 84.2) (width 0.75) (layer "F.Cu") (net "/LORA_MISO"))
 (segment (start 96 71.5) (end 104 79.5) (width 0.75) (layer "F.Cu") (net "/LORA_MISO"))
 (segment (start 85.5 71.5) (end 96 71.5) (width 0.75) (layer "F.Cu") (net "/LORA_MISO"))
 (segment (start 83.62 74.12) (end 83.62 73.38) (width 0.75) (layer "F.Cu") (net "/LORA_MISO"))
 (segment (start 86.16 74.12) (end 95.12 74.12) (width 0.75) (layer "F.Cu") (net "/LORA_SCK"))
 (segment (start 101.46 80.46) (end 101.46 84.2) (width 0.75) (layer "F.Cu") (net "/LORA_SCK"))
 (segment (start 95.12 74.12) (end 101.46 80.46) (width 0.75) (layer "F.Cu") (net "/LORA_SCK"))
 (segment (start 80.55 85.46) (end 77.54 85.46) (width 0.75) (layer "F.Cu") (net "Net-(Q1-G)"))
 (segment (start 76.08 91) (end 76.08 88.16) (width 0.75) (layer "F.Cu") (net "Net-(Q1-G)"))
 (segment (start 76 87) (end 76 88.08) (width 0.75) (layer "F.Cu") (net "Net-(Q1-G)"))
 (segment (start 77.54 85.46) (end 76 87) (width 0.75) (layer "F.Cu") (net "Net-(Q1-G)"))
 (segment (start 76.08 88.16) (end 76 88.08) (width 0.75) (layer "F.Cu") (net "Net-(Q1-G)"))
 (segment (start 110.5 90.5) (end 98.18 90.5) (width 1) (layer "F.Cu") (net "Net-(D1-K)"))
 (segment (start 110.5 90.5) (end 114.58 86.42) (width 1) (layer "F.Cu") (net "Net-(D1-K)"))
 (segment (start 98.18 90.5) (end 95.99 92.69) (width 1) (layer "F.Cu") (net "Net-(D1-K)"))
 (segment (start 87.5 92.69) (end 95.99 92.69) (width 1) (layer "F.Cu") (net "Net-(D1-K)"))
 (segment (start 114.58 86.42) (end 114.58 52) (width 1) (layer "F.Cu") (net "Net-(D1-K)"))
 (segment (start 96.95 93.65) (end 95.99 92.69) (width 1) (layer "F.Cu") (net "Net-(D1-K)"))
 (segment (start 96.95 95.05) (end 96.95 93.65) (width 1) (layer "F.Cu") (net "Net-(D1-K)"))
 (segment (start 82.5 88) (end 84 89.5) (width 0.75) (layer "F.Cu") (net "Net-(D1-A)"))
 (segment (start 87.5 104) (end 90.55 107.05) (width 0.75) (layer "F.Cu") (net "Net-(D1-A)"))
 (segment (start 90.55 107.05) (end 96.95 107.05) (width 0.75) (layer "F.Cu") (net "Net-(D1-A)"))
 (segment (start 84 100.5) (end 87.5 104) (width 0.75) (layer "F.Cu") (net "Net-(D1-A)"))
 (segment (start 87.5 104) (end 87.5 100.31) (width 0.75) (layer "F.Cu") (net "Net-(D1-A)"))
 (segment (start 84 89.5) (end 84 100.5) (width 0.75) (layer "F.Cu") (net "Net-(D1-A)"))
 (segment (start 80.55 88) (end 82.5 88) (width 0.75) (layer "F.Cu") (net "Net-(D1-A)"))
 (segment (start 122.5 90) (end 121 91.5) (width 1) (layer "F.Cu") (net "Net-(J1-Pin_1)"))
 (segment (start 122.5 49.75) (end 122.5 90) (width 1) (layer "F.Cu") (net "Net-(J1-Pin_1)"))
 (segment (start 121 91.5) (end 119.2175 91.5) (width 1) (layer "F.Cu") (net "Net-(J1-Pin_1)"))
 (segment (start 117.015 44.265) (end 122.5 49.75) (width 1) (layer "F.Cu") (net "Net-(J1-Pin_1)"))
 (segment (start 100.525 44.265) (end 117.015 44.265) (width 1) (layer "F.Cu") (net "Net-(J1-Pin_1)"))
 (segment (start 87 40) (end 89.5 37.5) (width 0.75) (layer "F.Cu") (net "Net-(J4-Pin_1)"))
 (segment (start 74.08 44.42) (end 78.5 40) (width 0.75) (layer "F.Cu") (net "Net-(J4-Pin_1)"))
 (segment (start 89.25 37.5) (end 89.5 37.5) (width 0.75) (layer "F.Cu") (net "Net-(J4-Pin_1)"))
 (segment (start 74 44.42) (end 74.08 44.42) (width 0.75) (layer "F.Cu") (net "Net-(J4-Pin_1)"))
 (segment (start 78.5 40) (end 87 40) (width 0.75) (layer "F.Cu") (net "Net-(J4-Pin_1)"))
 (segment (start 73.5 58.88) (end 73.5 55.08) (width 0.75) (layer "F.Cu") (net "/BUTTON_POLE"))
 (segment (start 73.5 55.08) (end 74 54.58) (width 0.75) (layer "F.Cu") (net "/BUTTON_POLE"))
 (segment (start 95 101) (end 125.16 101) (width 3.5) (layer "F.Cu") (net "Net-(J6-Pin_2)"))
 (segment (start 125.16 101) (end 125.35 101.19) (width 3.5) (layer "F.Cu") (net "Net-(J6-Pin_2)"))
 (segment (start 110.91 108.81) (end 109.15 107.05) (width 3.5) (layer "F.Cu") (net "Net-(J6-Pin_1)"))
 (segment (start 125.35 108.81) (end 110.91 108.81) (width 3.5) (layer "F.Cu") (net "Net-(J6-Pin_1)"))
 (segment (start 56.5 51.25) (end 57.75 50) (width 0.75) (layer "F.Cu") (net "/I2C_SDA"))
 (segment (start 56.5 58) (end 56.5 51.25) (width 0.75) (layer "F.Cu") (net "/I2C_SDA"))
 (segment (start 70.92 72.42) (end 56.5 58) (width 0.75) (layer "F.Cu") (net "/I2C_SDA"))
 (segment (start 70.92 74.12) (end 70.92 72.42) (width 0.75) (layer "F.Cu") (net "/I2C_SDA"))
 (segment (start 57.75 50) (end 59 50) (width 0.75) (layer "F.Cu") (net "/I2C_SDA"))
 (segment (start 59 57) (end 73.46 71.46) (width 0.75) (layer "F.Cu") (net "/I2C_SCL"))
 (segment (start 59 52.5) (end 59 57) (width 0.75) (layer "F.Cu") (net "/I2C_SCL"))
 (segment (start 73.46 71.46) (end 73.46 74.12) (width 0.75) (layer "F.Cu") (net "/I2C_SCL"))
 (segment (start 76 77.92) (end 76 74.12) (width 0.75) (layer "F.Cu") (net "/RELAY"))
 (segment (start 78.54 58.88) (end 78.54 58.04) (width 0.75) (layer "F.Cu") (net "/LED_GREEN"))
 (segment (start 78.54 58.04) (end 83 53.58) (width 0.75) (layer "F.Cu") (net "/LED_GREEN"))
 (segment (start 76 58.88) (end 76 57.08) (width 0.75) (layer "F.Cu") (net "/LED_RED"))
 (segment (start 76 57.08) (end 78.5 54.58) (width 0.75) (layer "F.Cu") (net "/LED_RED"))
 (segment (start 66.5 55.08) (end 68.38 56.96) (width 1) (layer "F.Cu") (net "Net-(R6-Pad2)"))
 (segment (start 68.38 56.96) (end 68.38 58.88) (width 1) (layer "F.Cu") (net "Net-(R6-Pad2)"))
 (segment (start 60.5 85.5) (end 68.38 77.62) (width 0.75) (layer "F.Cu") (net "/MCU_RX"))
 (segment (start 57.5 85.5) (end 60.5 85.5) (width 0.75) (layer "F.Cu") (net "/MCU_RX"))
 (segment (start 68.38 77.62) (end 68.38 74.12) (width 0.75) (layer "F.Cu") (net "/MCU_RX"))
 (segment (start 65.84 76.66) (end 65.84 74.12) (width 0.75) (layer "F.Cu") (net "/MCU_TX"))
 (segment (start 59.5 83) (end 65.84 76.66) (width 0.75) (layer "F.Cu") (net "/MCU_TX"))
 (segment (start 57.5 83) (end 59.5 83) (width 0.75) (layer "F.Cu") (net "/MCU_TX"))
 (segment (start 78.5 44.42) (end 80.58 46.5) (width 0.75) (layer "F.Cu") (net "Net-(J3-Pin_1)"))
 (segment (start 88.5 46.5) (end 89.5 45.5) (width 0.75) (layer "F.Cu") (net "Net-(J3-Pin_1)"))
 (segment (start 80.58 46.5) (end 88.5 46.5) (width 0.75) (layer "F.Cu") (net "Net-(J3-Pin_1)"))
 (segment (start 93 42.5) (end 94.5 44) (width 0.75) (layer "F.Cu") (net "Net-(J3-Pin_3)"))
 (segment (start 94.5 44) (end 94.5 45.5) (width 0.75) (layer "F.Cu") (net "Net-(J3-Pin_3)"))
 (segment (start 83 43.42) (end 83.92 42.5) (width 0.75) (layer "F.Cu") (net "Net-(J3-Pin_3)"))
 (segment (start 83.92 42.5) (end 93 42.5) (width 0.75) (layer "F.Cu") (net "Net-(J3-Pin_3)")))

